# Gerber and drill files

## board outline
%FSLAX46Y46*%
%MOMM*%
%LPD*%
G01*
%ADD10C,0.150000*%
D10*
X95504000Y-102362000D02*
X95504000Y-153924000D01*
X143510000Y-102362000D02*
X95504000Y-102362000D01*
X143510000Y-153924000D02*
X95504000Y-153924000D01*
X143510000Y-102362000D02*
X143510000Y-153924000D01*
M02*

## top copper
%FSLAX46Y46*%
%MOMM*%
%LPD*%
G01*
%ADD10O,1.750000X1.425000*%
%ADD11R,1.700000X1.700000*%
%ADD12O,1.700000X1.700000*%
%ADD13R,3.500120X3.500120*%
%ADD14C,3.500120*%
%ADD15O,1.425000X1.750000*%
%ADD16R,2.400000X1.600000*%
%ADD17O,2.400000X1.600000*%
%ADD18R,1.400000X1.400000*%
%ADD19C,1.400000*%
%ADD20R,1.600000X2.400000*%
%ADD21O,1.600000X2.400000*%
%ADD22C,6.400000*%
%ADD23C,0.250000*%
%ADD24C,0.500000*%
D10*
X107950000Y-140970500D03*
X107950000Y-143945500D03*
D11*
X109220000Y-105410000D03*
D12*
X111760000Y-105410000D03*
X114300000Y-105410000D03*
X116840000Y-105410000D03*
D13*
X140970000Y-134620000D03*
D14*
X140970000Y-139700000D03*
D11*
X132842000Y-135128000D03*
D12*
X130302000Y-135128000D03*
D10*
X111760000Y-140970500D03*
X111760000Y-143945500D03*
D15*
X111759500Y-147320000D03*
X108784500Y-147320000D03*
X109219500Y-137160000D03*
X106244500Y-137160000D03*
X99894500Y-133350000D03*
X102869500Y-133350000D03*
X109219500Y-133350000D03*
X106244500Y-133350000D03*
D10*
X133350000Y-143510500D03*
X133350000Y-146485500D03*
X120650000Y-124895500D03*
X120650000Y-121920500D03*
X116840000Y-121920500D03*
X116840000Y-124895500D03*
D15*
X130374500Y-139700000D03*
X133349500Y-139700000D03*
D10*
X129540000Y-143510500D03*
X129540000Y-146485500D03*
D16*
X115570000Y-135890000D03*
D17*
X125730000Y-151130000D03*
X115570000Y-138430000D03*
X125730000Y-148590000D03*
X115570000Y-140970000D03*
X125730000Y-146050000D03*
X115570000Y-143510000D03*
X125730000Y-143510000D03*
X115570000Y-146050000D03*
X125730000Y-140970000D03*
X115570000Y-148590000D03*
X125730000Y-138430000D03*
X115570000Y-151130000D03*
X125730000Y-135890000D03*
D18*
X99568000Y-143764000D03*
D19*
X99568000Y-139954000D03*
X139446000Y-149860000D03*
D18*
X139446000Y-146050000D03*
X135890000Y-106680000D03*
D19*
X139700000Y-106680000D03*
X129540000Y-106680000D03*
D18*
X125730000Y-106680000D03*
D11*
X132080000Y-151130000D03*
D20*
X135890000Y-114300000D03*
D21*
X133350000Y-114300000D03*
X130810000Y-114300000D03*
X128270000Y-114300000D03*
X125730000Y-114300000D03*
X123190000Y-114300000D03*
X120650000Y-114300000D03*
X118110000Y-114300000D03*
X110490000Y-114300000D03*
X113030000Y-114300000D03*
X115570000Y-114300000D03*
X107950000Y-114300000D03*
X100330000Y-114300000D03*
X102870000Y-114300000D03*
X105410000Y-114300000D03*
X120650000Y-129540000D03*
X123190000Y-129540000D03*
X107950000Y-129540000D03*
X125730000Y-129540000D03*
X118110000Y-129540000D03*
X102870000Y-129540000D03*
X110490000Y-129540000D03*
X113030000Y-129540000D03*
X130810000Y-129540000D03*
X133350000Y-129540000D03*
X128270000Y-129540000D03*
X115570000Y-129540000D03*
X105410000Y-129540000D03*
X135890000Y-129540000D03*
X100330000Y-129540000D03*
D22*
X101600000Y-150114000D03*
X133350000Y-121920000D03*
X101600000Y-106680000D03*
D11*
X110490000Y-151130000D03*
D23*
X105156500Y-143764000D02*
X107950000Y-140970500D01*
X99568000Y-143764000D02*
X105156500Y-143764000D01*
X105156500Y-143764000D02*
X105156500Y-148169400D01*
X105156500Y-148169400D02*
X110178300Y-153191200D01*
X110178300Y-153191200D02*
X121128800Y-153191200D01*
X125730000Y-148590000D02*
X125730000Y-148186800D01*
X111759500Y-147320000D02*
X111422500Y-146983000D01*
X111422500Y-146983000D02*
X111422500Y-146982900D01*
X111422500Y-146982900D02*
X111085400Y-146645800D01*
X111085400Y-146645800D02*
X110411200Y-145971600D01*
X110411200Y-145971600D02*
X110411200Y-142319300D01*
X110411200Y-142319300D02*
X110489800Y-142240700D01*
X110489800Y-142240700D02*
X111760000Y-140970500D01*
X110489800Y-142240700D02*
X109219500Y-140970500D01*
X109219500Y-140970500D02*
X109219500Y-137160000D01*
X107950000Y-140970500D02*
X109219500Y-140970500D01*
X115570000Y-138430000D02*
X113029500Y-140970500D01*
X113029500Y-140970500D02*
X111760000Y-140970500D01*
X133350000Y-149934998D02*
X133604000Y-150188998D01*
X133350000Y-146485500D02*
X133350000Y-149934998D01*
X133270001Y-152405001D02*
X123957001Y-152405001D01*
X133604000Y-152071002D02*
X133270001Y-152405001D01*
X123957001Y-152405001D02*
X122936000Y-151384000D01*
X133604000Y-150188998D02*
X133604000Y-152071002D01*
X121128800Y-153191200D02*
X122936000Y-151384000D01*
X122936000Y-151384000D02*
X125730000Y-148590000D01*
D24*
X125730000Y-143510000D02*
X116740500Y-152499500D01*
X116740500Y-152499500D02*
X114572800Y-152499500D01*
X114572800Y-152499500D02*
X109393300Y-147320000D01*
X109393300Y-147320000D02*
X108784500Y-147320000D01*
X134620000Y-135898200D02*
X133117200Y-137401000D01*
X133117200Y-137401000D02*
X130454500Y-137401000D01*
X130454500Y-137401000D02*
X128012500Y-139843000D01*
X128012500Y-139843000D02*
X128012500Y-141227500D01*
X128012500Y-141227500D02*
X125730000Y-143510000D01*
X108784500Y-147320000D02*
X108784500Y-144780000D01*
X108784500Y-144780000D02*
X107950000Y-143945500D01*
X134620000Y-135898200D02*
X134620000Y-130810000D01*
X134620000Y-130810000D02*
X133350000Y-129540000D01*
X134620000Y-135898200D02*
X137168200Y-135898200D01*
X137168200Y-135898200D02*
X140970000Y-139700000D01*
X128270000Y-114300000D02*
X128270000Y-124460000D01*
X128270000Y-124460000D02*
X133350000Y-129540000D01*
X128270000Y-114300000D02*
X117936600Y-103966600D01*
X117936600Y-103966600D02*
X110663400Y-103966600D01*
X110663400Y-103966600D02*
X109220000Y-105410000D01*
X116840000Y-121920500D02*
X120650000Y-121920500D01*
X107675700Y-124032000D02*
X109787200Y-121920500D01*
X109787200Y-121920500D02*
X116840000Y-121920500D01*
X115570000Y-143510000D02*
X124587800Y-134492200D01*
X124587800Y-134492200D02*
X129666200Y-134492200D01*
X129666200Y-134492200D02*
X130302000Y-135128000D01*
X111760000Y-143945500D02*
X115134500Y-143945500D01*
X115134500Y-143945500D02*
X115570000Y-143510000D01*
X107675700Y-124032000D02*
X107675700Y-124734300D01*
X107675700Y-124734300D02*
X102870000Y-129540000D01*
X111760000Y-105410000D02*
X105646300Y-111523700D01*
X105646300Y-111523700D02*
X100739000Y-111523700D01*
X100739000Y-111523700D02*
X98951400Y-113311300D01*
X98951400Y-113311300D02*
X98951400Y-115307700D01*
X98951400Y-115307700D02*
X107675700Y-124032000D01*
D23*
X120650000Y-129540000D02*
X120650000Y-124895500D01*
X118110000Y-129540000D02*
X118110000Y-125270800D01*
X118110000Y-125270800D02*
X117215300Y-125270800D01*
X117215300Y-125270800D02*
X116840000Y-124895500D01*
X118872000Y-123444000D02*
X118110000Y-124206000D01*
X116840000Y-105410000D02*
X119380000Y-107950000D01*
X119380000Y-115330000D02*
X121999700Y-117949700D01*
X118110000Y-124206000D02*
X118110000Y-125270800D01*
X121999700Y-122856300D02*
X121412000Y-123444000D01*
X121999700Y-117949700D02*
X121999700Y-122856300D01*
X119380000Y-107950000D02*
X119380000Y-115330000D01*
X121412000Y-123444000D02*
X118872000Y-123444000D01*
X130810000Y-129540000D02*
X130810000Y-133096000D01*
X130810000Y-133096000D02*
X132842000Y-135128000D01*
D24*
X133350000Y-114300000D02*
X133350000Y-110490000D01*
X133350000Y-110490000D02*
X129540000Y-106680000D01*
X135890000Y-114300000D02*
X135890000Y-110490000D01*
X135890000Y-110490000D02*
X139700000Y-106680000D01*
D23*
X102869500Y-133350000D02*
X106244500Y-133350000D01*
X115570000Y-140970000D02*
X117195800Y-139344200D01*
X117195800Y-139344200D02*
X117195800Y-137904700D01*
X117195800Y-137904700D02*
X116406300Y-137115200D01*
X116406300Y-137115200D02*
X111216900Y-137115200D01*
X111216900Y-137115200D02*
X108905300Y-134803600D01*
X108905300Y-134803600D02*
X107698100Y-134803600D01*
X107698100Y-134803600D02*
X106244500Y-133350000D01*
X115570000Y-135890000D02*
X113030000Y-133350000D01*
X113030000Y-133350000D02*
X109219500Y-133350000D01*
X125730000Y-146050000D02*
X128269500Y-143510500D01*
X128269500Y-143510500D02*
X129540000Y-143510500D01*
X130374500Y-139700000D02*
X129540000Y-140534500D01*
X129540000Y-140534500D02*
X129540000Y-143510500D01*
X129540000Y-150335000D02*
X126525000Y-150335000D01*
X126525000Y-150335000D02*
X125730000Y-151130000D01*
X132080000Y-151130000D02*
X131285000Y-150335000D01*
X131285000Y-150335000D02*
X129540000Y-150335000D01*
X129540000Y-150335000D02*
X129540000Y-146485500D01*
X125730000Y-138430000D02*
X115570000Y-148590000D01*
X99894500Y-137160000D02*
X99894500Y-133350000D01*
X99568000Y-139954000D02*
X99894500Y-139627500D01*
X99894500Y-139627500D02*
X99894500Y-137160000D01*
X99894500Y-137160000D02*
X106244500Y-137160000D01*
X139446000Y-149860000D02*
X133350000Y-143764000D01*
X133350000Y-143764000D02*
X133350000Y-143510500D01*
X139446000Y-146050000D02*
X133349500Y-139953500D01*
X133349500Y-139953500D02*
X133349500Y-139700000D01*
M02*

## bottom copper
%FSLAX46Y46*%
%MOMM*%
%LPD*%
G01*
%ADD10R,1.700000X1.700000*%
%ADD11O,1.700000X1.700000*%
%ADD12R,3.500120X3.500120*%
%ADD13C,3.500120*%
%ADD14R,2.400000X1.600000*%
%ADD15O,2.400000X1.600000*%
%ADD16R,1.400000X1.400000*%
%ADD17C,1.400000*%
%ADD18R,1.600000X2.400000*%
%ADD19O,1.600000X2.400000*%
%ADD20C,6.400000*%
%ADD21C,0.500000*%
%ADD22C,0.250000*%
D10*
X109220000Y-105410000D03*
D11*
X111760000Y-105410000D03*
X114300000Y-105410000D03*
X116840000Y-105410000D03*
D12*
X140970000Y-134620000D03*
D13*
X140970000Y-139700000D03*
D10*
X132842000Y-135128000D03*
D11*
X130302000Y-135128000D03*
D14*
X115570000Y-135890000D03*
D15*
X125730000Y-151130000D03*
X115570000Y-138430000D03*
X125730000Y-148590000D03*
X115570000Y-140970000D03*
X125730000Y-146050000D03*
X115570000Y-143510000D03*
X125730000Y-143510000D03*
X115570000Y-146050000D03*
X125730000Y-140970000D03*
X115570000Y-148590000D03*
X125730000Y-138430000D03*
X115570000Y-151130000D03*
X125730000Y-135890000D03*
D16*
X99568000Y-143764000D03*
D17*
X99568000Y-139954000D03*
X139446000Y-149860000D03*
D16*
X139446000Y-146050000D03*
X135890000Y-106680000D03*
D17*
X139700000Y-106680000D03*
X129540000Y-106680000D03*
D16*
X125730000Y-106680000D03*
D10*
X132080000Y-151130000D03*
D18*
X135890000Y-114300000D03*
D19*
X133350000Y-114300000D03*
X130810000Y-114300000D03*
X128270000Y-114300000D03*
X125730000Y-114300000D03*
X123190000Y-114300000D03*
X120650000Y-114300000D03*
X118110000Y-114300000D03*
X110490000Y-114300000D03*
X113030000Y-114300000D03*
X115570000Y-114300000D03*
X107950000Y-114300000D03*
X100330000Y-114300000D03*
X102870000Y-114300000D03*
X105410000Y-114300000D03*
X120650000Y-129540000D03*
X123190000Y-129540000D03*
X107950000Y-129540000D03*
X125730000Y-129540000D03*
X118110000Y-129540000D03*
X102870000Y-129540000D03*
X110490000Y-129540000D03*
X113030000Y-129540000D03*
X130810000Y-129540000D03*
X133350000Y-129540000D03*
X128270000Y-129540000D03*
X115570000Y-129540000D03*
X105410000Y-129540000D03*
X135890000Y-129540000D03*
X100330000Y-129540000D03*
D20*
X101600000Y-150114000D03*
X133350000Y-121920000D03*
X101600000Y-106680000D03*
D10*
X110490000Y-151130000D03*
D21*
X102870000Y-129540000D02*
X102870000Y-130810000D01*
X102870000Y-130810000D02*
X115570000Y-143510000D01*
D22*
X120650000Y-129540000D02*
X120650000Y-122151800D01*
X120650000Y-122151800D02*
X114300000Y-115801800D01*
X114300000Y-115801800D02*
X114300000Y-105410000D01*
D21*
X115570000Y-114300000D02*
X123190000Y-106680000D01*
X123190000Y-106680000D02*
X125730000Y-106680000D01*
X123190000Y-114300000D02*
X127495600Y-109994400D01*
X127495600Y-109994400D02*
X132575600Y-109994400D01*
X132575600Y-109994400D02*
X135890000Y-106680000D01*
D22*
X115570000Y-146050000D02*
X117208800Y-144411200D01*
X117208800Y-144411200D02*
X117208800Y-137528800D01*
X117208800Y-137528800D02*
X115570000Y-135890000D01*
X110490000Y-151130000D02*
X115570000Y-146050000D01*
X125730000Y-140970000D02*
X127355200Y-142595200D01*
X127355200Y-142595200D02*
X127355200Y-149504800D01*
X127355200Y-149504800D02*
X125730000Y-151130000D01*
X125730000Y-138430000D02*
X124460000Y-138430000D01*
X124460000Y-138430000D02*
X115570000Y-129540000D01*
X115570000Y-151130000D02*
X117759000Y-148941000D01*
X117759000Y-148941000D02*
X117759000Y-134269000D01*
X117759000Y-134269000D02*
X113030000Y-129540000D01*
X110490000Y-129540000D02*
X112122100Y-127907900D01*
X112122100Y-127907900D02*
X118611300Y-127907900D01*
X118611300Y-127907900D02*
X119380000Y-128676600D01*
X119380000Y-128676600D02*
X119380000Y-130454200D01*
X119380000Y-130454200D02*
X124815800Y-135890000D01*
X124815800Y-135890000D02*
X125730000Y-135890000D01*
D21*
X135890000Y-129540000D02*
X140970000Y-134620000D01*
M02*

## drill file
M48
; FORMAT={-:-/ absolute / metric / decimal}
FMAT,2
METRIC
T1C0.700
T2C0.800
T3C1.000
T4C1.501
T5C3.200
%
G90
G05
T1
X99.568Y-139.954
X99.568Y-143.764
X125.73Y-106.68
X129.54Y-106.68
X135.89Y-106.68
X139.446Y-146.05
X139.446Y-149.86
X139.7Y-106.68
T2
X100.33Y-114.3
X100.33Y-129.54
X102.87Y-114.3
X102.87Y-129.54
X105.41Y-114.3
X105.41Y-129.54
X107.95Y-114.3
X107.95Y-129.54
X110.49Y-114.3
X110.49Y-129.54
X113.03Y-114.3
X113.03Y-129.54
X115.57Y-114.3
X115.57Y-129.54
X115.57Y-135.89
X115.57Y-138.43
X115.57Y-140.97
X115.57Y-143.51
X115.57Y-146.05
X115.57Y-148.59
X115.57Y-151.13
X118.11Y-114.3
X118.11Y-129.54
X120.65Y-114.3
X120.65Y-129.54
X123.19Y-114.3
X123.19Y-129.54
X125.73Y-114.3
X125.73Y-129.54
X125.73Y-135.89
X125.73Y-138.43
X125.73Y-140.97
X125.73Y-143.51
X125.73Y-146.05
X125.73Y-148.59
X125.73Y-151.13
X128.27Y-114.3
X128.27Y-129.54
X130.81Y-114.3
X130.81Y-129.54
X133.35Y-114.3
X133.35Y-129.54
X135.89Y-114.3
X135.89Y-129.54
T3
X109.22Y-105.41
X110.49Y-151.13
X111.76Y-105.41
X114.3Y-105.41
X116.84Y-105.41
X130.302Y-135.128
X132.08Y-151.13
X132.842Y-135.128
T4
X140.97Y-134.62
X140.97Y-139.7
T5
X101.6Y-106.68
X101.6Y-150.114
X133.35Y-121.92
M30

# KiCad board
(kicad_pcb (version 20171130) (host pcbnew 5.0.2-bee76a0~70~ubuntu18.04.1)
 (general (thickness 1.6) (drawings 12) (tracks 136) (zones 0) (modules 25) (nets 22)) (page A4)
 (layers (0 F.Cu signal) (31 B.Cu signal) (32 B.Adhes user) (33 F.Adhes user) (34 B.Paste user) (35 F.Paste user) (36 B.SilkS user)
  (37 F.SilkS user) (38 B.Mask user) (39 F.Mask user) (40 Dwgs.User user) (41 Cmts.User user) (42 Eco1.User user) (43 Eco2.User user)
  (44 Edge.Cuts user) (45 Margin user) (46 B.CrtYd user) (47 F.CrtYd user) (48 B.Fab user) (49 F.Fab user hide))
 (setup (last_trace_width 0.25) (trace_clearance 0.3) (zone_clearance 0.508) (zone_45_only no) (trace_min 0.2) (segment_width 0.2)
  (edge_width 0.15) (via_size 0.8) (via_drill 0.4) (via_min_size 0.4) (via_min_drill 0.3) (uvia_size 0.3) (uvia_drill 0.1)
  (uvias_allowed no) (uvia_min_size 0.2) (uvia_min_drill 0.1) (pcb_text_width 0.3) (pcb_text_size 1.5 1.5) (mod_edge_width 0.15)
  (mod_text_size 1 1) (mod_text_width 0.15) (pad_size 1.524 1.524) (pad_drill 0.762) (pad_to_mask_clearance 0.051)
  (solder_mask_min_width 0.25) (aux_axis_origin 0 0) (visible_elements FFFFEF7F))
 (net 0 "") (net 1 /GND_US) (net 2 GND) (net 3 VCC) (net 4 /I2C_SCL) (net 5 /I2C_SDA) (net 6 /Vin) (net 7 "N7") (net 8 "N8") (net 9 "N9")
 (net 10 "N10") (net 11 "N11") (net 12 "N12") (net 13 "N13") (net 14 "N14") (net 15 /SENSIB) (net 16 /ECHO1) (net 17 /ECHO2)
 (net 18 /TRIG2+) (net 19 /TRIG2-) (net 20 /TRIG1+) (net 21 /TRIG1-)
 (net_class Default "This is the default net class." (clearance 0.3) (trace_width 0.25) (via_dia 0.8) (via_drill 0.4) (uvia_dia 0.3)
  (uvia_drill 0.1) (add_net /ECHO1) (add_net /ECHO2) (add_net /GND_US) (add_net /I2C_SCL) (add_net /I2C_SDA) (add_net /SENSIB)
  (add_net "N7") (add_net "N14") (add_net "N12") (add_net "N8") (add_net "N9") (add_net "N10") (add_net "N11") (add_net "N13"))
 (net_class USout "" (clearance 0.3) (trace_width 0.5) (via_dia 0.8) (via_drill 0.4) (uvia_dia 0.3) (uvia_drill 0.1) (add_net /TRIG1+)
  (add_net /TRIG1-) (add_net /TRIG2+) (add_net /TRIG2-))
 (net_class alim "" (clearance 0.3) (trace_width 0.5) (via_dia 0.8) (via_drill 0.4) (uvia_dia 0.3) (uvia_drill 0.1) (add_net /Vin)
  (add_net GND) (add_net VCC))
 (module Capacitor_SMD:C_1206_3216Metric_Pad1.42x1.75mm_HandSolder (layer F.Cu) (at 107.95 142.458 270)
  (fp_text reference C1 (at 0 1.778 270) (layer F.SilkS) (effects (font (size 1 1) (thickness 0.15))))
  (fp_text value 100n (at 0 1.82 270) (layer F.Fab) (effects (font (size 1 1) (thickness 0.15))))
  (pad 1 smd oval (at -1.4875 0 270) (size 1.425 1.75) (layers F.Cu F.Paste F.Mask) (roundrect_rratio 0.175439) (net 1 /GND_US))
  (pad 2 smd oval (at 1.4875 0 270) (size 1.425 1.75) (layers F.Cu F.Paste F.Mask) (roundrect_rratio 0.175439) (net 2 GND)))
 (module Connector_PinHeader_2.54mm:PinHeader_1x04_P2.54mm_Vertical (layer F.Cu) (at 109.22 105.41 90)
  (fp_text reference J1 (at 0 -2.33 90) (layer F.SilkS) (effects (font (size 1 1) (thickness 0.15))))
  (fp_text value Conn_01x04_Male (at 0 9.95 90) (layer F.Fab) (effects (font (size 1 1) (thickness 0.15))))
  (pad 1 thru_hole rect (at 0 0 90) (size 1.7 1.7) (drill 1) (layers *.Cu *.Mask) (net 2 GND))
  (pad 2 thru_hole oval (at 0 2.54 90) (size 1.7 1.7) (drill 1) (layers *.Cu *.Mask) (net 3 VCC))
  (pad 3 thru_hole oval (at 0 5.08 90) (size 1.7 1.7) (drill 1) (layers *.Cu *.Mask) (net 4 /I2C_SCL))
  (pad 4 thru_hole oval (at 0 7.62 90) (size 1.7 1.7) (drill 1) (layers *.Cu *.Mask) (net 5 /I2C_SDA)))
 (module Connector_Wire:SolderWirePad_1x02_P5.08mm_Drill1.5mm (layer F.Cu) (at 140.97 134.62 270)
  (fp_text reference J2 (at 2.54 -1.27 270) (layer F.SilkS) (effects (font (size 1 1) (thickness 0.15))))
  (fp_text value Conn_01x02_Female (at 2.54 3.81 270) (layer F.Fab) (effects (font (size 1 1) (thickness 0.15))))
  (pad 1 thru_hole rect (at 0 0 270) (size 3.50012 3.50012) (drill 1.50114) (layers *.Cu *.Mask) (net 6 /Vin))
  (pad 2 thru_hole circle (at 5.08 0 270) (size 3.50012 3.50012) (drill 1.50114) (layers *.Cu *.Mask) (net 2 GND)))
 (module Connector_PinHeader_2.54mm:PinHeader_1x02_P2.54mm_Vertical (layer F.Cu) (at 132.842 135.128 270)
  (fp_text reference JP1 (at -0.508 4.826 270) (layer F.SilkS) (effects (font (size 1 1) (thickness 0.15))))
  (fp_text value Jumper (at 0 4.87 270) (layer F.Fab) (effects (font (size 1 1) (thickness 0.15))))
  (pad 1 thru_hole rect (at 0 0 270) (size 1.7 1.7) (drill 1) (layers *.Cu *.Mask) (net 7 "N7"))
  (pad 2 thru_hole oval (at 0 2.54 270) (size 1.7 1.7) (drill 1) (layers *.Cu *.Mask) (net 3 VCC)))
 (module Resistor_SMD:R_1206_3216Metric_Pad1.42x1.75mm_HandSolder (layer F.Cu) (at 111.76 142.458 90)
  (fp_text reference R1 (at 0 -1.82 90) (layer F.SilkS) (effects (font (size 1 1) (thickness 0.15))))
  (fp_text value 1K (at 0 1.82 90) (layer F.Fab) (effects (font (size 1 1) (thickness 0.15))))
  (pad 2 smd oval (at 1.4875 0 90) (size 1.425 1.75) (layers F.Cu F.Paste F.Mask) (roundrect_rratio 0.175439) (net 1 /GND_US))
  (pad 1 smd oval (at -1.4875 0 90) (size 1.425 1.75) (layers F.Cu F.Paste F.Mask) (roundrect_rratio 0.175439) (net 3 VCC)))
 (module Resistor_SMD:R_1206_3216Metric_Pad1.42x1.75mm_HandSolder (layer F.Cu) (at 110.272 147.32 180)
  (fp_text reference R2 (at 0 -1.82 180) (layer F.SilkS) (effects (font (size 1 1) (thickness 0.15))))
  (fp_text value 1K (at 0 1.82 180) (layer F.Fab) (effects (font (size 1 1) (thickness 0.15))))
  (pad 1 smd oval (at -1.4875 0 180) (size 1.425 1.75) (layers F.Cu F.Paste F.Mask) (roundrect_rratio 0.175439) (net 1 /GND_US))
  (pad 2 smd oval (at 1.4875 0 180) (size 1.425 1.75) (layers F.Cu F.Paste F.Mask) (roundrect_rratio 0.175439) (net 2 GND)))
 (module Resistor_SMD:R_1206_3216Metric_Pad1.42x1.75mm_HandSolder (layer F.Cu) (at 107.732 137.16 180)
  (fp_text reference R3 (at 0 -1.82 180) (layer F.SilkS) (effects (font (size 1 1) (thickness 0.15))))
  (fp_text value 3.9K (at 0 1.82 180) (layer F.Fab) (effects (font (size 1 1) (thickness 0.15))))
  (pad 1 smd oval (at -1.4875 0 180) (size 1.425 1.75) (layers F.Cu F.Paste F.Mask) (roundrect_rratio 0.175439) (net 1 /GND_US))
  (pad 2 smd oval (at 1.4875 0 180) (size 1.425 1.75) (layers F.Cu F.Paste F.Mask) (roundrect_rratio 0.175439) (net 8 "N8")))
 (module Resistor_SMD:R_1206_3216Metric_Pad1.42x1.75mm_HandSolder (layer F.Cu) (at 101.382 133.35 180)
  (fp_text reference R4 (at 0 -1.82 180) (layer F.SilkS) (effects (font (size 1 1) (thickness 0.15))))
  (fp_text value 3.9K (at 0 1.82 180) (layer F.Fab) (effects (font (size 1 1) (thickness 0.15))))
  (pad 2 smd oval (at 1.4875 0 180) (size 1.425 1.75) (layers F.Cu F.Paste F.Mask) (roundrect_rratio 0.175439) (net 8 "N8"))
  (pad 1 smd oval (at -1.4875 0 180) (size 1.425 1.75) (layers F.Cu F.Paste F.Mask) (roundrect_rratio 0.175439) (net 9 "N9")))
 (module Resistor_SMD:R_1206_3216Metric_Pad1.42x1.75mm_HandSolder (layer F.Cu) (at 107.732 133.35 180)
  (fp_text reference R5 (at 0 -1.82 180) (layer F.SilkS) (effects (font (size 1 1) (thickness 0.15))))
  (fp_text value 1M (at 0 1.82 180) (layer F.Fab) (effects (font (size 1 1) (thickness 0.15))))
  (pad 1 smd oval (at -1.4875 0 180) (size 1.425 1.75) (layers F.Cu F.Paste F.Mask) (roundrect_rratio 0.175439) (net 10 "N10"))
  (pad 2 smd oval (at 1.4875 0 180) (size 1.425 1.75) (layers F.Cu F.Paste F.Mask) (roundrect_rratio 0.175439) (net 9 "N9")))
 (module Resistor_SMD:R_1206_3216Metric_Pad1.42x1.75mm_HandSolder (layer F.Cu) (at 133.35 144.998 90)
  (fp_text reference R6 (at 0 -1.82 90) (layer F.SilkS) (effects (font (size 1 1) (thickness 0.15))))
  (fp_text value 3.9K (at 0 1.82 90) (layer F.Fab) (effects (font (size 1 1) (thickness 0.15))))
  (pad 2 smd oval (at 1.4875 0 90) (size 1.425 1.75) (layers F.Cu F.Paste F.Mask) (roundrect_rratio 0.175439) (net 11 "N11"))
  (pad 1 smd oval (at -1.4875 0 90) (size 1.425 1.75) (layers F.Cu F.Paste F.Mask) (roundrect_rratio 0.175439) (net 1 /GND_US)))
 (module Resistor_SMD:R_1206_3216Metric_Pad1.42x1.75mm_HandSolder (layer F.Cu) (at 120.65 123.408 90)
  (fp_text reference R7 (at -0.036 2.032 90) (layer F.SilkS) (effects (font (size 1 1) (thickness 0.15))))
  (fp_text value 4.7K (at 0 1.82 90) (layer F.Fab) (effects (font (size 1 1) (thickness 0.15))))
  (pad 1 smd oval (at -1.4875 0 90) (size 1.425 1.75) (layers F.Cu F.Paste F.Mask) (roundrect_rratio 0.175439) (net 4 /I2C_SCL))
  (pad 2 smd oval (at 1.4875 0 90) (size 1.425 1.75) (layers F.Cu F.Paste F.Mask) (roundrect_rratio 0.175439) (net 3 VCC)))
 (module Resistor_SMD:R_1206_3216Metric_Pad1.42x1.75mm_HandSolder (layer F.Cu) (at 116.84 123.408 90)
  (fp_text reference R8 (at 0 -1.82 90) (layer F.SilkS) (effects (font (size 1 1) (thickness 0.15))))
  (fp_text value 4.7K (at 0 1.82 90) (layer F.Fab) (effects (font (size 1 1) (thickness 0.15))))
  (pad 2 smd oval (at 1.4875 0 90) (size 1.425 1.75) (layers F.Cu F.Paste F.Mask) (roundrect_rratio 0.175439) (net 3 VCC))
  (pad 1 smd oval (at -1.4875 0 90) (size 1.425 1.75) (layers F.Cu F.Paste F.Mask) (roundrect_rratio 0.175439) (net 5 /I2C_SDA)))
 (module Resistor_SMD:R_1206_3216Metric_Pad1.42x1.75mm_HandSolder (layer F.Cu) (at 131.862 139.7)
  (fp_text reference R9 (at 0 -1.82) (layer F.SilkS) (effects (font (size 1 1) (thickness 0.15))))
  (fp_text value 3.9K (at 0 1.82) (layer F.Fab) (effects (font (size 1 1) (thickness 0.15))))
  (pad 1 smd oval (at -1.4875 0) (size 1.425 1.75) (layers F.Cu F.Paste F.Mask) (roundrect_rratio 0.175439) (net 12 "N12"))
  (pad 2 smd oval (at 1.4875 0) (size 1.425 1.75) (layers F.Cu F.Paste F.Mask) (roundrect_rratio 0.175439) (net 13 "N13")))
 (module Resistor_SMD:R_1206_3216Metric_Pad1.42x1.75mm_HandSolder (layer F.Cu) (at 129.54 144.998 90)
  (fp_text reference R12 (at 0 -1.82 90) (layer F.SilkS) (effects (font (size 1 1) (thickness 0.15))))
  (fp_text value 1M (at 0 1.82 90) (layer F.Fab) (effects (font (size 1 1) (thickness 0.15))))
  (pad 2 smd oval (at 1.4875 0 90) (size 1.425 1.75) (layers F.Cu F.Paste F.Mask) (roundrect_rratio 0.175439) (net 12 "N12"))
  (pad 1 smd oval (at -1.4875 0 90) (size 1.425 1.75) (layers F.Cu F.Paste F.Mask) (roundrect_rratio 0.175439) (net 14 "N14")))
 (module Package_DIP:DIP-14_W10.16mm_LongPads (layer F.Cu) (at 115.57 135.89)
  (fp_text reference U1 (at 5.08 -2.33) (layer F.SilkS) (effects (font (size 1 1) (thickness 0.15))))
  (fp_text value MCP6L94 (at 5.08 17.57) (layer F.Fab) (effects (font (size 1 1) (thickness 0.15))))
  (pad 1 thru_hole rect (at 0 0) (size 2.4 1.6) (drill 0.8) (layers *.Cu *.Mask) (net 10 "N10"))
  (pad 8 thru_hole oval (at 10.16 15.24) (size 2.4 1.6) (drill 0.8) (layers *.Cu *.Mask) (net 14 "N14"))
  (pad 2 thru_hole oval (at 0 2.54) (size 2.4 1.6) (drill 0.8) (layers *.Cu *.Mask) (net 1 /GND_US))
  (pad 9 thru_hole oval (at 10.16 12.7) (size 2.4 1.6) (drill 0.8) (layers *.Cu *.Mask) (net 1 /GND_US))
  (pad 3 thru_hole oval (at 0 5.08) (size 2.4 1.6) (drill 0.8) (layers *.Cu *.Mask) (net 9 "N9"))
  (pad 10 thru_hole oval (at 10.16 10.16) (size 2.4 1.6) (drill 0.8) (layers *.Cu *.Mask) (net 12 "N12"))
  (pad 4 thru_hole oval (at 0 7.62) (size 2.4 1.6) (drill 0.8) (layers *.Cu *.Mask) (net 3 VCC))
  (pad 11 thru_hole oval (at 10.16 7.62) (size 2.4 1.6) (drill 0.8) (layers *.Cu *.Mask) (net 2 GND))
  (pad 5 thru_hole oval (at 0 10.16) (size 2.4 1.6) (drill 0.8) (layers *.Cu *.Mask) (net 10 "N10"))
  (pad 12 thru_hole oval (at 10.16 5.08) (size 2.4 1.6) (drill 0.8) (layers *.Cu *.Mask) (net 14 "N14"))
  (pad 6 thru_hole oval (at 0 12.7) (size 2.4 1.6) (drill 0.8) (layers *.Cu *.Mask) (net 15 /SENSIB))
  (pad 13 thru_hole oval (at 10.16 2.54) (size 2.4 1.6) (drill 0.8) (layers *.Cu *.Mask) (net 15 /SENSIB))
  (pad 7 thru_hole oval (at 0 15.24) (size 2.4 1.6) (drill 0.8) (layers *.Cu *.Mask) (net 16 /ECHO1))
  (pad 14 thru_hole oval (at 10.16 0) (size 2.4 1.6) (drill 0.8) (layers *.Cu *.Mask) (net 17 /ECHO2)))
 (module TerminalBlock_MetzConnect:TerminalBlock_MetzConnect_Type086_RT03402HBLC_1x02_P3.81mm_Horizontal (layer F.Cu) (at 99.568 143.764 90)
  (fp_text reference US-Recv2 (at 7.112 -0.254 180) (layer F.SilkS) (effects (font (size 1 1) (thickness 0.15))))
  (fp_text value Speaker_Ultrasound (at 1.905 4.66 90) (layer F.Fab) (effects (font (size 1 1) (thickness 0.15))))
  (pad 1 thru_hole rect (at 0 0 90) (size 1.4 1.4) (drill 0.7) (layers *.Cu *.Mask) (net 1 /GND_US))
  (pad 2 thru_hole circle (at 3.81 0 90) (size 1.4 1.4) (drill 0.7) (layers *.Cu *.Mask) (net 8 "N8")))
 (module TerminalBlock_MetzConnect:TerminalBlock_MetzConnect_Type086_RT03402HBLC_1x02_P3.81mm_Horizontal (layer F.Cu)
  (at 139.446 146.05 270)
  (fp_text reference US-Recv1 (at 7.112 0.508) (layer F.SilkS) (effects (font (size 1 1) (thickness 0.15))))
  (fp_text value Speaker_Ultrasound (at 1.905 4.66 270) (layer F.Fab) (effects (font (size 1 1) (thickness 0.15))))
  (pad 2 thru_hole circle (at 3.81 0 270) (size 1.4 1.4) (drill 0.7) (layers *.Cu *.Mask) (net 11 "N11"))
  (pad 1 thru_hole rect (at 0 0 270) (size 1.4 1.4) (drill 0.7) (layers *.Cu *.Mask) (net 13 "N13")))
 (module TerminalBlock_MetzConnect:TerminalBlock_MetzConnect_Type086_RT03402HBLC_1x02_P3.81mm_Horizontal (layer F.Cu) (at 135.89 106.68)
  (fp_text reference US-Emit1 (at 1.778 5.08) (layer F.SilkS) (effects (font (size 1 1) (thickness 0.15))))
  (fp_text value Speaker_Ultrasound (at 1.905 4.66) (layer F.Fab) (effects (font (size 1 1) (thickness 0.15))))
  (pad 1 thru_hole rect (at 0 0) (size 1.4 1.4) (drill 0.7) (layers *.Cu *.Mask) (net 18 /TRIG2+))
  (pad 2 thru_hole circle (at 3.81 0) (size 1.4 1.4) (drill 0.7) (layers *.Cu *.Mask) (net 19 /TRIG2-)))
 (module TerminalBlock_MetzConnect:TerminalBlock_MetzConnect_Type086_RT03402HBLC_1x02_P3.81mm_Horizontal (layer F.Cu) (at 125.73 106.68)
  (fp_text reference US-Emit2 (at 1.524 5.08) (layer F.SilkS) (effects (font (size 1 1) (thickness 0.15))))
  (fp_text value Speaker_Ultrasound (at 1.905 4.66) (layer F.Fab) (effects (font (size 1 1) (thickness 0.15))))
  (pad 2 thru_hole circle (at 3.81 0) (size 1.4 1.4) (drill 0.7) (layers *.Cu *.Mask) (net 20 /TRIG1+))
  (pad 1 thru_hole rect (at 0 0) (size 1.4 1.4) (drill 0.7) (layers *.Cu *.Mask) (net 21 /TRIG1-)))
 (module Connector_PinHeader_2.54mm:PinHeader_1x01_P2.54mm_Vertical (layer F.Cu) (at 132.08 151.13)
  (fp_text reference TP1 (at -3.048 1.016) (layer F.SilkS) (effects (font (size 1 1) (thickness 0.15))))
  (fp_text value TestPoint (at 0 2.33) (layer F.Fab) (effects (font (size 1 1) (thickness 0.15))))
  (pad 1 thru_hole rect (at 0 0) (size 1.7 1.7) (drill 1) (layers *.Cu *.Mask) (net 14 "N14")))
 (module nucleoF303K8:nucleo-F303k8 (layer F.Cu) (at 135.89 121.92 270)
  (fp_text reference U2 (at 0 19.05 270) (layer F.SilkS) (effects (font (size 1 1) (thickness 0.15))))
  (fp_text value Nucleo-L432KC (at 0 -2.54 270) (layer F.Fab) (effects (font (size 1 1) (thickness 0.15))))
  (pad 1 thru_hole rect (at -7.62 0 270) (size 2.4 1.6) (drill 0.8) (layers *.Cu *.Mask) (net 19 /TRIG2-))
  (pad 2 thru_hole oval (at -7.62 2.54 270) (size 2.4 1.6) (drill 0.8) (layers *.Cu *.Mask) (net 20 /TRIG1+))
  (pad 3 thru_hole oval (at -7.62 5.08 270) (size 2.4 1.6) (drill 0.8) (layers *.Cu *.Mask))
  (pad 4 thru_hole oval (at -7.62 7.62 270) (size 2.4 1.6) (drill 0.8) (layers *.Cu *.Mask) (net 2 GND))
  (pad 5 thru_hole oval (at -7.62 10.16 270) (size 2.4 1.6) (drill 0.8) (layers *.Cu *.Mask))
  (pad 6 thru_hole oval (at -7.62 12.7 270) (size 2.4 1.6) (drill 0.8) (layers *.Cu *.Mask) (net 18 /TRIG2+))
  (pad 7 thru_hole oval (at -7.62 15.24 270) (size 2.4 1.6) (drill 0.8) (layers *.Cu *.Mask))
  (pad 8 thru_hole oval (at -7.62 17.78 270) (size 2.4 1.6) (drill 0.8) (layers *.Cu *.Mask))
  (pad 11 thru_hole oval (at -7.62 25.4 270) (size 2.4 1.6) (drill 0.8) (layers *.Cu *.Mask))
  (pad 10 thru_hole oval (at -7.62 22.86 270) (size 2.4 1.6) (drill 0.8) (layers *.Cu *.Mask))
  (pad 9 thru_hole oval (at -7.62 20.32 270) (size 2.4 1.6) (drill 0.8) (layers *.Cu *.Mask) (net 21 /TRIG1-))
  (pad 12 thru_hole oval (at -7.62 27.94 270) (size 2.4 1.6) (drill 0.8) (layers *.Cu *.Mask))
  (pad 15 thru_hole oval (at -7.62 35.56 270) (size 2.4 1.6) (drill 0.8) (layers *.Cu *.Mask))
  (pad 14 thru_hole oval (at -7.62 33.02 270) (size 2.4 1.6) (drill 0.8) (layers *.Cu *.Mask))
  (pad 13 thru_hole oval (at -7.62 30.48 270) (size 2.4 1.6) (drill 0.8) (layers *.Cu *.Mask))
  (pad 24 thru_hole oval (at 7.62 15.24 270) (size 2.4 1.6) (drill 0.8) (layers *.Cu *.Mask) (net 4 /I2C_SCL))
  (pad 25 thru_hole oval (at 7.62 12.7 270) (size 2.4 1.6) (drill 0.8) (layers *.Cu *.Mask))
  (pad 19 thru_hole oval (at 7.62 27.94 270) (size 2.4 1.6) (drill 0.8) (layers *.Cu *.Mask))
  (pad 26 thru_hole oval (at 7.62 10.16 270) (size 2.4 1.6) (drill 0.8) (layers *.Cu *.Mask))
  (pad 23 thru_hole oval (at 7.62 17.78 270) (size 2.4 1.6) (drill 0.8) (layers *.Cu *.Mask) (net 5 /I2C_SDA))
  (pad 17 thru_hole oval (at 7.62 33.02 270) (size 2.4 1.6) (drill 0.8) (layers *.Cu *.Mask) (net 3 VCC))
  (pad 20 thru_hole oval (at 7.62 25.4 270) (size 2.4 1.6) (drill 0.8) (layers *.Cu *.Mask) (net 17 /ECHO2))
  (pad 21 thru_hole oval (at 7.62 22.86 270) (size 2.4 1.6) (drill 0.8) (layers *.Cu *.Mask) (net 16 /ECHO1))
  (pad 28 thru_hole oval (at 7.62 5.08 270) (size 2.4 1.6) (drill 0.8) (layers *.Cu *.Mask) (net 7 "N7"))
  (pad 29 thru_hole oval (at 7.62 2.54 270) (size 2.4 1.6) (drill 0.8) (layers *.Cu *.Mask) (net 2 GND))
  (pad 27 thru_hole oval (at 7.62 7.62 270) (size 2.4 1.6) (drill 0.8) (layers *.Cu *.Mask))
  (pad 22 thru_hole oval (at 7.62 20.32 270) (size 2.4 1.6) (drill 0.8) (layers *.Cu *.Mask) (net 15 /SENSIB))
  (pad 18 thru_hole oval (at 7.62 30.48 270) (size 2.4 1.6) (drill 0.8) (layers *.Cu *.Mask))
  (pad 30 thru_hole oval (at 7.62 0 270) (size 2.4 1.6) (drill 0.8) (layers *.Cu *.Mask) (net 6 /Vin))
  (pad 16 thru_hole oval (at 7.62 35.56 270) (size 2.4 1.6) (drill 0.8) (layers *.Cu *.Mask)))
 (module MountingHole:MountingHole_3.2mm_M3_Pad (layer F.Cu) (at 101.6 150.114)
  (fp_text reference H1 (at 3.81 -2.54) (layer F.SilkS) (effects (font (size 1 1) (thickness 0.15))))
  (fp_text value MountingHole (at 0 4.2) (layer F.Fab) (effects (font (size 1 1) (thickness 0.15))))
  (pad 1 thru_hole circle (at 0 0) (size 6.4 6.4) (drill 3.2) (layers *.Cu *.Mask)))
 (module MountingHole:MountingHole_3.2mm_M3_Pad (layer F.Cu) (at 133.35 121.92)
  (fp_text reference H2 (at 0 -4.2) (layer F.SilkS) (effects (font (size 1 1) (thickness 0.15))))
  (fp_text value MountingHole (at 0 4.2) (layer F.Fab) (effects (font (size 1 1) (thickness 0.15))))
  (pad 1 thru_hole circle (at 0 0) (size 6.4 6.4) (drill 3.2) (layers *.Cu *.Mask)))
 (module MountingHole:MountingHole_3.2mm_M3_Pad (layer F.Cu) (at 101.6 106.68)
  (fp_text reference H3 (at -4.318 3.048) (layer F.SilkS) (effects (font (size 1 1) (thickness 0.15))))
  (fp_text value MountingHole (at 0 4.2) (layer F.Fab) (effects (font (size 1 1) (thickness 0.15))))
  (pad 1 thru_hole circle (at 0 0) (size 6.4 6.4) (drill 3.2) (layers *.Cu *.Mask)))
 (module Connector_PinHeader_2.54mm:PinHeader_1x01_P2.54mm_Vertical (layer F.Cu) (at 110.49 151.13)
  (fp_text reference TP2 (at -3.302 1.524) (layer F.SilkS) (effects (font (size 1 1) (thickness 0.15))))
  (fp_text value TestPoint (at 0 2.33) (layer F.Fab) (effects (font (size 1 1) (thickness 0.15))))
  (pad 1 thru_hole rect (at 0 0) (size 1.7 1.7) (drill 1) (layers *.Cu *.Mask) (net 10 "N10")))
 (gr_line (start 95.504 102.362) (end 95.504 153.924) (layer Edge.Cuts) (width 0.15))
 (gr_line (start 143.51 102.362) (end 95.504 102.362) (layer Edge.Cuts) (width 0.15))
 (gr_line (start 143.51 153.924) (end 95.504 153.924) (layer Edge.Cuts) (width 0.15))
 (gr_line (start 143.51 102.362) (end 143.51 153.924) (layer Edge.Cuts) (width 0.15))
 (segment (start 105.1565 143.764) (end 107.95 140.9705) (width 0.25) (layer F.Cu) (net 1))
 (segment (start 99.568 143.764) (end 105.1565 143.764) (width 0.25) (layer F.Cu) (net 1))
 (segment (start 105.1565 143.764) (end 105.1565 148.1694) (width 0.25) (layer F.Cu) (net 1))
 (segment (start 105.1565 148.1694) (end 110.1783 153.1912) (width 0.25) (layer F.Cu) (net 1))
 (segment (start 110.1783 153.1912) (end 121.1288 153.1912) (width 0.25) (layer F.Cu) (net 1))
 (segment (start 125.73 148.59) (end 125.73 148.1868) (width 0.25) (layer F.Cu) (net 1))
 (segment (start 111.7595 147.32) (end 111.4225 146.983) (width 0.25) (layer F.Cu) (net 1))
 (segment (start 111.4225 146.983) (end 111.4225 146.9829) (width 0.25) (layer F.Cu) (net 1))
 (segment (start 111.4225 146.9829) (end 111.0854 146.6458) (width 0.25) (layer F.Cu) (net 1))
 (segment (start 111.0854 146.6458) (end 110.4112 145.9716) (width 0.25) (layer F.Cu) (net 1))
 (segment (start 110.4112 145.9716) (end 110.4112 142.3193) (width 0.25) (layer F.Cu) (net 1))
 (segment (start 110.4112 142.3193) (end 110.4898 142.2407) (width 0.25) (layer F.Cu) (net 1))
 (segment (start 110.4898 142.2407) (end 111.76 140.9705) (width 0.25) (layer F.Cu) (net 1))
 (segment (start 110.4898 142.2407) (end 109.2195 140.9705) (width 0.25) (layer F.Cu) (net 1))
 (segment (start 109.2195 140.9705) (end 109.2195 137.16) (width 0.25) (layer F.Cu) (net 1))
 (segment (start 107.95 140.9705) (end 109.2195 140.9705) (width 0.25) (layer F.Cu) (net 1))
 (segment (start 115.57 138.43) (end 113.0295 140.9705) (width 0.25) (layer F.Cu) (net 1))
 (segment (start 113.0295 140.9705) (end 111.76 140.9705) (width 0.25) (layer F.Cu) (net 1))
 (segment (start 133.35 149.934998) (end 133.604 150.188998) (width 0.25) (layer F.Cu) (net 1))
 (segment (start 133.35 146.4855) (end 133.35 149.934998) (width 0.25) (layer F.Cu) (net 1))
 (segment (start 133.270001 152.405001) (end 123.957001 152.405001) (width 0.25) (layer F.Cu) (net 1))
 (segment (start 133.604 152.071002) (end 133.270001 152.405001) (width 0.25) (layer F.Cu) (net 1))
 (segment (start 123.957001 152.405001) (end 122.936 151.384) (width 0.25) (layer F.Cu) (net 1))
 (segment (start 133.604 150.188998) (end 133.604 152.071002) (width 0.25) (layer F.Cu) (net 1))
 (segment (start 121.1288 153.1912) (end 122.936 151.384) (width 0.25) (layer F.Cu) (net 1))
 (segment (start 122.936 151.384) (end 125.73 148.59) (width 0.25) (layer F.Cu) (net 1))
 (segment (start 125.73 143.51) (end 116.7405 152.4995) (width 0.5) (layer F.Cu) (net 2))
 (segment (start 116.7405 152.4995) (end 114.5728 152.4995) (width 0.5) (layer F.Cu) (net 2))
 (segment (start 114.5728 152.4995) (end 109.3933 147.32) (width 0.5) (layer F.Cu) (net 2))
 (segment (start 109.3933 147.32) (end 108.7845 147.32) (width 0.5) (layer F.Cu) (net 2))
 (segment (start 134.62 135.8982) (end 133.1172 137.401) (width 0.5) (layer F.Cu) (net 2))
 (segment (start 133.1172 137.401) (end 130.4545 137.401) (width 0.5) (layer F.Cu) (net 2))
 (segment (start 130.4545 137.401) (end 128.0125 139.843) (width 0.5) (layer F.Cu) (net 2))
 (segment (start 128.0125 139.843) (end 128.0125 141.2275) (width 0.5) (layer F.Cu) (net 2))
 (segment (start 128.0125 141.2275) (end 125.73 143.51) (width 0.5) (layer F.Cu) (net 2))
 (segment (start 108.7845 147.32) (end 108.7845 144.78) (width 0.5) (layer F.Cu) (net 2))
 (segment (start 108.7845 144.78) (end 107.95 143.9455) (width 0.5) (layer F.Cu) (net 2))
 (segment (start 134.62 135.8982) (end 134.62 130.81) (width 0.5) (layer F.Cu) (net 2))
 (segment (start 134.62 130.81) (end 133.35 129.54) (width 0.5) (layer F.Cu) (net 2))
 (segment (start 134.62 135.8982) (end 137.1682 135.8982) (width 0.5) (layer F.Cu) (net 2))
 (segment (start 137.1682 135.8982) (end 140.97 139.7) (width 0.5) (layer F.Cu) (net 2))
 (segment (start 128.27 114.3) (end 128.27 124.46) (width 0.5) (layer F.Cu) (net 2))
 (segment (start 128.27 124.46) (end 133.35 129.54) (width 0.5) (layer F.Cu) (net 2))
 (segment (start 128.27 114.3) (end 117.9366 103.9666) (width 0.5) (layer F.Cu) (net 2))
 (segment (start 117.9366 103.9666) (end 110.6634 103.9666) (width 0.5) (layer F.Cu) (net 2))
 (segment (start 110.6634 103.9666) (end 109.22 105.41) (width 0.5) (layer F.Cu) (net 2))
 (segment (start 116.84 121.9205) (end 120.65 121.9205) (width 0.5) (layer F.Cu) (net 3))
 (segment (start 107.6757 124.032) (end 109.7872 121.9205) (width 0.5) (layer F.Cu) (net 3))
 (segment (start 109.7872 121.9205) (end 116.84 121.9205) (width 0.5) (layer F.Cu) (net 3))
 (segment (start 115.57 143.51) (end 124.5878 134.4922) (width 0.5) (layer F.Cu) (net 3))
 (segment (start 124.5878 134.4922) (end 129.6662 134.4922) (width 0.5) (layer F.Cu) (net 3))
 (segment (start 129.6662 134.4922) (end 130.302 135.128) (width 0.5) (layer F.Cu) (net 3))
 (segment (start 111.76 143.9455) (end 115.1345 143.9455) (width 0.5) (layer F.Cu) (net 3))
 (segment (start 115.1345 143.9455) (end 115.57 143.51) (width 0.5) (layer F.Cu) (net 3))
 (segment (start 102.87 129.54) (end 102.87 130.81) (width 0.5) (layer B.Cu) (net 3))
 (segment (start 102.87 130.81) (end 115.57 143.51) (width 0.5) (layer B.Cu) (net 3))
 (segment (start 107.6757 124.032) (end 107.6757 124.7343) (width 0.5) (layer F.Cu) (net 3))
 (segment (start 107.6757 124.7343) (end 102.87 129.54) (width 0.5) (layer F.Cu) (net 3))
 (segment (start 111.76 105.41) (end 105.6463 111.5237) (width 0.5) (layer F.Cu) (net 3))
 (segment (start 105.6463 111.5237) (end 100.739 111.5237) (width 0.5) (layer F.Cu) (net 3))
 (segment (start 100.739 111.5237) (end 98.9514 113.3113) (width 0.5) (layer F.Cu) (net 3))
 (segment (start 98.9514 113.3113) (end 98.9514 115.3077) (width 0.5) (layer F.Cu) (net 3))
 (segment (start 98.9514 115.3077) (end 107.6757 124.032) (width 0.5) (layer F.Cu) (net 3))
 (segment (start 120.65 129.54) (end 120.65 124.8955) (width 0.25) (layer F.Cu) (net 4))
 (segment (start 120.65 129.54) (end 120.65 122.1518) (width 0.25) (layer B.Cu) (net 4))
 (segment (start 120.65 122.1518) (end 114.3 115.8018) (width 0.25) (layer B.Cu) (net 4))
 (segment (start 114.3 115.8018) (end 114.3 105.41) (width 0.25) (layer B.Cu) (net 4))
 (segment (start 118.11 129.54) (end 118.11 125.2708) (width 0.25) (layer F.Cu) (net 5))
 (segment (start 118.11 125.2708) (end 117.2153 125.2708) (width 0.25) (layer F.Cu) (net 5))
 (segment (start 117.2153 125.2708) (end 116.84 124.8955) (width 0.25) (layer F.Cu) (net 5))
 (segment (start 118.872 123.444) (end 118.11 124.206) (width 0.25) (layer F.Cu) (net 5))
 (segment (start 116.84 105.41) (end 119.38 107.95) (width 0.25) (layer F.Cu) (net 5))
 (segment (start 119.38 115.33) (end 121.9997 117.9497) (width 0.25) (layer F.Cu) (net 5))
 (segment (start 118.11 124.206) (end 118.11 125.2708) (width 0.25) (layer F.Cu) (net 5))
 (segment (start 121.9997 122.8563) (end 121.412 123.444) (width 0.25) (layer F.Cu) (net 5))
 (segment (start 121.9997 117.9497) (end 121.9997 122.8563) (width 0.25) (layer F.Cu) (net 5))
 (segment (start 119.38 107.95) (end 119.38 115.33) (width 0.25) (layer F.Cu) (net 5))
 (segment (start 121.412 123.444) (end 118.872 123.444) (width 0.25) (layer F.Cu) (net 5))
 (segment (start 130.81 129.54) (end 130.81 133.096) (width 0.25) (layer F.Cu) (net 7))
 (segment (start 130.81 133.096) (end 132.842 135.128) (width 0.25) (layer F.Cu) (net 7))
 (segment (start 115.57 114.3) (end 123.19 106.68) (width 0.5) (layer B.Cu) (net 21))
 (segment (start 123.19 106.68) (end 125.73 106.68) (width 0.5) (layer B.Cu) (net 21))
 (segment (start 133.35 114.3) (end 133.35 110.49) (width 0.5) (layer F.Cu) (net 20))
 (segment (start 133.35 110.49) (end 129.54 106.68) (width 0.5) (layer F.Cu) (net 20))
 (segment (start 123.19 114.3) (end 127.4956 109.9944) (width 0.5) (layer B.Cu) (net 18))
 (segment (start 127.4956 109.9944) (end 132.5756 109.9944) (width 0.5) (layer B.Cu) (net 18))
 (segment (start 132.5756 109.9944) (end 135.89 106.68) (width 0.5) (layer B.Cu) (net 18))
 (segment (start 135.89 114.3) (end 135.89 110.49) (width 0.5) (layer F.Cu) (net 19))
 (segment (start 135.89 110.49) (end 139.7 106.68) (width 0.5) (layer F.Cu) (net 19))
 (segment (start 102.8695 133.35) (end 106.2445 133.35) (width 0.25) (layer F.Cu) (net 9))
 (segment (start 115.57 140.97) (end 117.1958 139.3442) (width 0.25) (layer F.Cu) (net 9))
 (segment (start 117.1958 139.3442) (end 117.1958 137.9047) (width 0.25) (layer F.Cu) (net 9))
 (segment (start 117.1958 137.9047) (end 116.4063 137.1152) (width 0.25) (layer F.Cu) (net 9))
 (segment (start 116.4063 137.1152) (end 111.2169 137.1152) (width 0.25) (layer F.Cu) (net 9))
 (segment (start 111.2169 137.1152) (end 108.9053 134.8036) (width 0.25) (layer F.Cu) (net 9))
 (segment (start 108.9053 134.8036) (end 107.6981 134.8036) (width 0.25) (layer F.Cu) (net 9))
 (segment (start 107.6981 134.8036) (end 106.2445 133.35) (width 0.25) (layer F.Cu) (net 9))
 (segment (start 115.57 146.05) (end 117.2088 144.4112) (width 0.25) (layer B.Cu) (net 10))
 (segment (start 117.2088 144.4112) (end 117.2088 137.5288) (width 0.25) (layer B.Cu) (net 10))
 (segment (start 117.2088 137.5288) (end 115.57 135.89) (width 0.25) (layer B.Cu) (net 10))
 (segment (start 110.49 151.13) (end 115.57 146.05) (width 0.25) (layer B.Cu) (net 10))
 (segment (start 115.57 135.89) (end 113.03 133.35) (width 0.25) (layer F.Cu) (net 10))
 (segment (start 113.03 133.35) (end 109.2195 133.35) (width 0.25) (layer F.Cu) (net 10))
 (segment (start 125.73 146.05) (end 128.2695 143.5105) (width 0.25) (layer F.Cu) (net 12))
 (segment (start 128.2695 143.5105) (end 129.54 143.5105) (width 0.25) (layer F.Cu) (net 12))
 (segment (start 130.3745 139.7) (end 129.54 140.5345) (width 0.25) (layer F.Cu) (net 12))
 (segment (start 129.54 140.5345) (end 129.54 143.5105) (width 0.25) (layer F.Cu) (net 12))
 (segment (start 125.73 140.97) (end 127.3552 142.5952) (width 0.25) (layer B.Cu) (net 14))
 (segment (start 127.3552 142.5952) (end 127.3552 149.5048) (width 0.25) (layer B.Cu) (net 14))
 (segment (start 127.3552 149.5048) (end 125.73 151.13) (width 0.25) (layer B.Cu) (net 14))
 (segment (start 129.54 150.335) (end 126.525 150.335) (width 0.25) (layer F.Cu) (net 14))
 (segment (start 126.525 150.335) (end 125.73 151.13) (width 0.25) (layer F.Cu) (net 14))
 (segment (start 132.08 151.13) (end 131.285 150.335) (width 0.25) (layer F.Cu) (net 14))
 (segment (start 131.285 150.335) (end 129.54 150.335) (width 0.25) (layer F.Cu) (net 14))
 (segment (start 129.54 150.335) (end 129.54 146.4855) (width 0.25) (layer F.Cu) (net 14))
 (segment (start 125.73 138.43) (end 115.57 148.59) (width 0.25) (layer F.Cu) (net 15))
 (segment (start 125.73 138.43) (end 124.46 138.43) (width 0.25) (layer B.Cu) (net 15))
 (segment (start 124.46 138.43) (end 115.57 129.54) (width 0.25) (layer B.Cu) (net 15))
 (segment (start 115.57 151.13) (end 117.759 148.941) (width 0.25) (layer B.Cu) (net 16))
 (segment (start 117.759 148.941) (end 117.759 134.269) (width 0.25) (layer B.Cu) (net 16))
 (segment (start 117.759 134.269) (end 113.03 129.54) (width 0.25) (layer B.Cu) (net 16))
 (segment (start 110.49 129.54) (end 112.1221 127.9079) (width 0.25) (layer B.Cu) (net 17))
 (segment (start 112.1221 127.9079) (end 118.6113 127.9079) (width 0.25) (layer B.Cu) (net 17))
 (segment (start 118.6113 127.9079) (end 119.38 128.6766) (width 0.25) (layer B.Cu) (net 17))
 (segment (start 119.38 128.6766) (end 119.38 130.4542) (width 0.25) (layer B.Cu) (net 17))
 (segment (start 119.38 130.4542) (end 124.8158 135.89) (width 0.25) (layer B.Cu) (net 17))
 (segment (start 124.8158 135.89) (end 125.73 135.89) (width 0.25) (layer B.Cu) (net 17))
 (segment (start 135.89 129.54) (end 140.97 134.62) (width 0.5) (layer B.Cu) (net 6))
 (segment (start 99.8945 137.16) (end 99.8945 133.35) (width 0.25) (layer F.Cu) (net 8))
 (segment (start 99.568 139.954) (end 99.8945 139.6275) (width 0.25) (layer F.Cu) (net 8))
 (segment (start 99.8945 139.6275) (end 99.8945 137.16) (width 0.25) (layer F.Cu) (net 8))
 (segment (start 99.8945 137.16) (end 106.2445 137.16) (width 0.25) (layer F.Cu) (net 8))
 (segment (start 139.446 149.86) (end 133.35 143.764) (width 0.25) (layer F.Cu) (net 11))
 (segment (start 133.35 143.764) (end 133.35 143.5105) (width 0.25) (layer F.Cu) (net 11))
 (segment (start 139.446 146.05) (end 133.3495 139.9535) (width 0.25) (layer F.Cu) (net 13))
 (segment (start 133.3495 139.9535) (end 133.3495 139.7) (width 0.25) (layer F.Cu) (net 13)))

